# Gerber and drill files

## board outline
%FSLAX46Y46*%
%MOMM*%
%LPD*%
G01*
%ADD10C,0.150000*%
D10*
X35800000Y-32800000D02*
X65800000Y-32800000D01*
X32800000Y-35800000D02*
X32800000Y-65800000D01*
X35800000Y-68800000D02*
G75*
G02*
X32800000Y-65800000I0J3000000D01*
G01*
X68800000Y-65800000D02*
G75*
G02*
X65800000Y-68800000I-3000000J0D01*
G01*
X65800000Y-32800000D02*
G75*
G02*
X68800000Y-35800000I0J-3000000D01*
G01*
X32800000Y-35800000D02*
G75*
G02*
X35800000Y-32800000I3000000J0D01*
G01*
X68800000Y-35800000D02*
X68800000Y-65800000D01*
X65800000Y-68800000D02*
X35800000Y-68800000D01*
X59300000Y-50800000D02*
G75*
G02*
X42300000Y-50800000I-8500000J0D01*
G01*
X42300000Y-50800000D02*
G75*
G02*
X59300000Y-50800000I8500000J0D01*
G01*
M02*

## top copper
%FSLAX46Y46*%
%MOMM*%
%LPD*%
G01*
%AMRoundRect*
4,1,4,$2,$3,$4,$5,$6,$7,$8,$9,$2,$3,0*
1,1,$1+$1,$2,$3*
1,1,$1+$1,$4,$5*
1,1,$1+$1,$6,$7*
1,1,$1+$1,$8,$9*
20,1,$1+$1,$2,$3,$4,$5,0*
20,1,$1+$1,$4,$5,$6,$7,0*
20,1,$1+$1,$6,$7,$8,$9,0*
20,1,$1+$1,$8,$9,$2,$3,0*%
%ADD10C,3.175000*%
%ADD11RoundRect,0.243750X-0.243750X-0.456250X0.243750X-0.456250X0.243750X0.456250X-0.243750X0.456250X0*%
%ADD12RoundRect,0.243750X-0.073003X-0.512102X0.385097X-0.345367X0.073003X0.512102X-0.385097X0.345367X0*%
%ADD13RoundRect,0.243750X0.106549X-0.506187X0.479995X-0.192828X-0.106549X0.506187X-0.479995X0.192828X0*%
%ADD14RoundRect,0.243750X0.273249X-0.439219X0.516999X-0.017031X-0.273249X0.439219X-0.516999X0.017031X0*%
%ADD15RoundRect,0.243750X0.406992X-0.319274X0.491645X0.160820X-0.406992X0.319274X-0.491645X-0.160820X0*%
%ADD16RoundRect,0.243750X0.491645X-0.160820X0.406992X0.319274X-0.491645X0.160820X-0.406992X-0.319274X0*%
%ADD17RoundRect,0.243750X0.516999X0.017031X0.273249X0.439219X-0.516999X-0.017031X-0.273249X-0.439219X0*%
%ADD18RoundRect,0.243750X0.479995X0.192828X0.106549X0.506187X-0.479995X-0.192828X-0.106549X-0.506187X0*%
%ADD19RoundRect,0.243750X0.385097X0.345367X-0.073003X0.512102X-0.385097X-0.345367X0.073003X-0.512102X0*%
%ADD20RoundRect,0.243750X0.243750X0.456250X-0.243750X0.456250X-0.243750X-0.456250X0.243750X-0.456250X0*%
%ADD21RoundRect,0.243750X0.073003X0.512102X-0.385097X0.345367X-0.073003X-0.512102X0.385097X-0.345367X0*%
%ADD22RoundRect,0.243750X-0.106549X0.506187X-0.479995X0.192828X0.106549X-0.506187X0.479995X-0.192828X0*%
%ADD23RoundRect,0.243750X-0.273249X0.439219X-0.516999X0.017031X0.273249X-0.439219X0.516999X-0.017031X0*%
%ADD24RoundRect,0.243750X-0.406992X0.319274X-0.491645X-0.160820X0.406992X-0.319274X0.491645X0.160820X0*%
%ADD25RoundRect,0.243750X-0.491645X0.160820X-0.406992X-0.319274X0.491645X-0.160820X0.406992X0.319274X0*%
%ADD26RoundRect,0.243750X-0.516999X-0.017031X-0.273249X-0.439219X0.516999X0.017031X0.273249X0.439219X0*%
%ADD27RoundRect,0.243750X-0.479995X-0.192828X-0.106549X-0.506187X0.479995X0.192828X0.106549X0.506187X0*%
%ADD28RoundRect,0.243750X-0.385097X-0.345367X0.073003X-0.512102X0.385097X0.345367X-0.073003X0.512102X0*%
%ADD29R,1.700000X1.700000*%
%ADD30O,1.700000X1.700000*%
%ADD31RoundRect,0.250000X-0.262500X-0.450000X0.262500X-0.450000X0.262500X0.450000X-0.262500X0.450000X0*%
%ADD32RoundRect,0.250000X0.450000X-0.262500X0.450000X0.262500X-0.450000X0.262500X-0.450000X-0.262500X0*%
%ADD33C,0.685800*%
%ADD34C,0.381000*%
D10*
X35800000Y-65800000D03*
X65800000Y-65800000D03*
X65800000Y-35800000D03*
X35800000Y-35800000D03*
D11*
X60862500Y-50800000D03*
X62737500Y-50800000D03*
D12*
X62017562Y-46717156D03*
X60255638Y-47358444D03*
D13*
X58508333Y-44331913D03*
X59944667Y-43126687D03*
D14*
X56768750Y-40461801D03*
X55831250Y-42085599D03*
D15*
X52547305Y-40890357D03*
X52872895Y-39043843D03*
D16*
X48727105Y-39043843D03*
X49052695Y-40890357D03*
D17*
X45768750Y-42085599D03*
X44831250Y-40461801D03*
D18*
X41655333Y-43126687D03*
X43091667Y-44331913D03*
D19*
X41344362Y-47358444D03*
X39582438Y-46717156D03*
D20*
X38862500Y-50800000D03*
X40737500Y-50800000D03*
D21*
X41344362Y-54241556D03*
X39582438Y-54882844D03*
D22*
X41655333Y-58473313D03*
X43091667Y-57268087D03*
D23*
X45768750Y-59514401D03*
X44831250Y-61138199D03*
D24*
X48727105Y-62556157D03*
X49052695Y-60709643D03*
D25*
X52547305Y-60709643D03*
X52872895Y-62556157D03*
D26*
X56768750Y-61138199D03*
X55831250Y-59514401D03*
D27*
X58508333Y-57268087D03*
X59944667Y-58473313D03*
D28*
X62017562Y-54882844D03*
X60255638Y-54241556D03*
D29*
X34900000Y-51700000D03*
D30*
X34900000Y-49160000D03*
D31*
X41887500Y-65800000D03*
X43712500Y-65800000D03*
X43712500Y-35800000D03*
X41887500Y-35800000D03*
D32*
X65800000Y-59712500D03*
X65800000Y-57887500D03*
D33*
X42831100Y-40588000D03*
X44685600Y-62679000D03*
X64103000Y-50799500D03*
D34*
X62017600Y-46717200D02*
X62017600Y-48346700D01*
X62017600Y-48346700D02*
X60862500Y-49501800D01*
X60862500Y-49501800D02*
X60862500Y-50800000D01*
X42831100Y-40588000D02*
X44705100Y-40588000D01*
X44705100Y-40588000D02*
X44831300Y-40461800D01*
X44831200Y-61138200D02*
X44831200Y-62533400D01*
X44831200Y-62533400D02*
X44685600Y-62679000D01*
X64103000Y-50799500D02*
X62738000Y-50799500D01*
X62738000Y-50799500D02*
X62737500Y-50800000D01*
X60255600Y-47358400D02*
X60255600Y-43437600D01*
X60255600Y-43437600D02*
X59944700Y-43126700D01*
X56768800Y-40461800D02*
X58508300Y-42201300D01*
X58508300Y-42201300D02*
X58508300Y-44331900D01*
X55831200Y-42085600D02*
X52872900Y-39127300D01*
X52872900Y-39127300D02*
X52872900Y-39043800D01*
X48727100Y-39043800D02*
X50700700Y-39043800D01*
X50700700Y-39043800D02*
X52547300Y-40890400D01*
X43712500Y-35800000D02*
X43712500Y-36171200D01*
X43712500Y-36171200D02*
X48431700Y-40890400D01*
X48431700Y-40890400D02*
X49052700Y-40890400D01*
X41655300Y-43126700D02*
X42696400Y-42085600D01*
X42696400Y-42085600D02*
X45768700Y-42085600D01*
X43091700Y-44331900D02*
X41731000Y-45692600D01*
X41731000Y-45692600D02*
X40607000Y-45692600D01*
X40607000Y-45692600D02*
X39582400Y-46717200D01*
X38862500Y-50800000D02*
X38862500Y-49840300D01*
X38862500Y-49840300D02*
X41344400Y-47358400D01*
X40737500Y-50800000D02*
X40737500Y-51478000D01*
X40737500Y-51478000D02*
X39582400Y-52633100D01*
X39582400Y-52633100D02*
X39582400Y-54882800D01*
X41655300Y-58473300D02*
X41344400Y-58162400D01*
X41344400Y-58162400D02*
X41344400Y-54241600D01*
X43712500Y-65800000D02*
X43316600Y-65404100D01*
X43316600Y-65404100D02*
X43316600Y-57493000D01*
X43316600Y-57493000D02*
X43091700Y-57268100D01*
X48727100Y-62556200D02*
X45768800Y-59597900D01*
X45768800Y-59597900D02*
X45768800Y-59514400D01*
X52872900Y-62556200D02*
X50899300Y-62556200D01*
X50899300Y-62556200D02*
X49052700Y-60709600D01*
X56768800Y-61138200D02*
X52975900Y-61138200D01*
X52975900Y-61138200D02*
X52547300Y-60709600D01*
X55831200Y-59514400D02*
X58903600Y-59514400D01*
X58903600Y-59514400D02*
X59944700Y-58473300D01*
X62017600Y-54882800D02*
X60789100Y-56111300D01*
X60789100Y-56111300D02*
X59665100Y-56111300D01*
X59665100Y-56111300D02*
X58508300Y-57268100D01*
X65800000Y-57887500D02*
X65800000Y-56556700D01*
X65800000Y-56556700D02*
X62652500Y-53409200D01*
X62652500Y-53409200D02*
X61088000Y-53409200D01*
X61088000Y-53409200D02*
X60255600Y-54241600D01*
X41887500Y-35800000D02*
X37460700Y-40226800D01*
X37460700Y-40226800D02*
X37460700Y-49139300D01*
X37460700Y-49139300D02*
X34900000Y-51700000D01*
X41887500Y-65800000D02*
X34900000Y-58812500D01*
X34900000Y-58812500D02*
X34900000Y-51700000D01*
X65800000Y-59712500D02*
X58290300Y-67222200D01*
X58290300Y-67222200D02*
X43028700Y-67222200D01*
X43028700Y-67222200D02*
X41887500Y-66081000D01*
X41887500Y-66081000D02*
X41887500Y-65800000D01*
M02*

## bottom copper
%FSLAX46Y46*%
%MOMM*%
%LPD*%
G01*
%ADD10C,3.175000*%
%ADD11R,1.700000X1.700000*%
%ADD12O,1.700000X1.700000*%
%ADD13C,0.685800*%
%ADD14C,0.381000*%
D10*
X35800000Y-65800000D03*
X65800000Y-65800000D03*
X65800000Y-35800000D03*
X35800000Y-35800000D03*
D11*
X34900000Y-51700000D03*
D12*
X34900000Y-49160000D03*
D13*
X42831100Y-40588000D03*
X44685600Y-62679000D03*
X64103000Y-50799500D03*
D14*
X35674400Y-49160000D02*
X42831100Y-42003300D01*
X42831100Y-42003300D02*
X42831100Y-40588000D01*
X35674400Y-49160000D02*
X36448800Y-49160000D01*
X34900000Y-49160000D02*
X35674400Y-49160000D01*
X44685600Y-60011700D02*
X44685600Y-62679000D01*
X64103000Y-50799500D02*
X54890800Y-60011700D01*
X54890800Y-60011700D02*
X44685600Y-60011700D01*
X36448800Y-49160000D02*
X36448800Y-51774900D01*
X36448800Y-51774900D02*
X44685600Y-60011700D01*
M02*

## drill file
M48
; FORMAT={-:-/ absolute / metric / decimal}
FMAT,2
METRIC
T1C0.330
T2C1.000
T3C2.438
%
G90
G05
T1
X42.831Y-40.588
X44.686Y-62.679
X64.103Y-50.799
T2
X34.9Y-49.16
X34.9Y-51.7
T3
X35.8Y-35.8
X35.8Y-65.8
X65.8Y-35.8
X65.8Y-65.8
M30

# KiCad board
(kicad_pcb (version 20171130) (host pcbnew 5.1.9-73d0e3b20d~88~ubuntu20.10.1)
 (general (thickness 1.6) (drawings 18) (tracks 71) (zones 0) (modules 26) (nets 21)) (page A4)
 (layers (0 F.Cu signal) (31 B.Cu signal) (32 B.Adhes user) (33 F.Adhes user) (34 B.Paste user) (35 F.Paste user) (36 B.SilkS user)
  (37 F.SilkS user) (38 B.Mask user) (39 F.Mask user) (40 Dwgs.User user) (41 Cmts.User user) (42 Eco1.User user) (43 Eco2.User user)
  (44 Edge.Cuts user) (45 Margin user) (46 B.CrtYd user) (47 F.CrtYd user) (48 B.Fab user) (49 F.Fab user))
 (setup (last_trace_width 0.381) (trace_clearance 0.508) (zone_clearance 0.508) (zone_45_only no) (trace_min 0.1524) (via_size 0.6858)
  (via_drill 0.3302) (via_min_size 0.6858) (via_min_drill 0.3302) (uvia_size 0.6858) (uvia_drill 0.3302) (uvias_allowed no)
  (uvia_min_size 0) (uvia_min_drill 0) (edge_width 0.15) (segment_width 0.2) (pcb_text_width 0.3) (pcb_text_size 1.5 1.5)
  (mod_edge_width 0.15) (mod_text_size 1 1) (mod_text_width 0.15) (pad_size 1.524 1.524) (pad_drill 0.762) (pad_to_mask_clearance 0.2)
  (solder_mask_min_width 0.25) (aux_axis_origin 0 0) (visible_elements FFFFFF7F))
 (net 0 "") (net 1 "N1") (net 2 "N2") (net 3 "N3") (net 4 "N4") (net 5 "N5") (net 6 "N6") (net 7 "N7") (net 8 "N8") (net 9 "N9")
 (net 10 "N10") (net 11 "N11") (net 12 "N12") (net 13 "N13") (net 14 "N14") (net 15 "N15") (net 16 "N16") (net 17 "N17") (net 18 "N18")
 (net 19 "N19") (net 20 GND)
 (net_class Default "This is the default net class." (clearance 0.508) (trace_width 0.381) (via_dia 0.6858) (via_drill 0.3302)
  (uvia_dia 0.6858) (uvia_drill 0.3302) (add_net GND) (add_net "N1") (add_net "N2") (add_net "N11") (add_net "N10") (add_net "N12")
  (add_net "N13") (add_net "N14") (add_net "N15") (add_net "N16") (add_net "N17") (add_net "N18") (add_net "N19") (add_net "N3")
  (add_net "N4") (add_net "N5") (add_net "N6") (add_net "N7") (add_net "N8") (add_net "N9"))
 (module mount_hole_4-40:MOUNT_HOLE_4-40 (layer F.Cu) (at 35.8 65.8)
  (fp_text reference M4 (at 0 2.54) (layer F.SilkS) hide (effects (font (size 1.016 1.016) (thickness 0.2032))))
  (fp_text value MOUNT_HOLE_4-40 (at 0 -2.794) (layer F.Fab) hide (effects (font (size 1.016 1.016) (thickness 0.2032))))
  (pad 1 thru_hole circle (at 0 0) (size 3.175 3.175) (drill 2.4384) (layers *.Cu *.Mask)))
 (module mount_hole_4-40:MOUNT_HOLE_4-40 (layer F.Cu) (at 65.8 65.8)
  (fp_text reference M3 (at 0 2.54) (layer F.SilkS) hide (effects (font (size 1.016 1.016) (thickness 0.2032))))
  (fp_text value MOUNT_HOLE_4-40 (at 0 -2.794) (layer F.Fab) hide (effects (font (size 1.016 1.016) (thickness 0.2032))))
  (pad 1 thru_hole circle (at 0 0) (size 3.175 3.175) (drill 2.4384) (layers *.Cu *.Mask)))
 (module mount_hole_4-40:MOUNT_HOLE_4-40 (layer F.Cu) (at 65.8 35.8)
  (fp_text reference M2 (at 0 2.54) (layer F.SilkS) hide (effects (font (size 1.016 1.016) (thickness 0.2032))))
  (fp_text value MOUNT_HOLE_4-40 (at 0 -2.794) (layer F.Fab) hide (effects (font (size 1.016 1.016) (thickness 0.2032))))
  (pad 1 thru_hole circle (at 0 0) (size 3.175 3.175) (drill 2.4384) (layers *.Cu *.Mask)))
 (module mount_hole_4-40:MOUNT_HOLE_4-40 (layer F.Cu) (at 35.8 35.8)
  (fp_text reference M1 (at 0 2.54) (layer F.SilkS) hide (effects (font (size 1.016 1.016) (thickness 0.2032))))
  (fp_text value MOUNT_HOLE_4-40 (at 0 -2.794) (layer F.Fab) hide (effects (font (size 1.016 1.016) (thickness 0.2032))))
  (pad 1 thru_hole circle (at 0 0) (size 3.175 3.175) (drill 2.4384) (layers *.Cu *.Mask)))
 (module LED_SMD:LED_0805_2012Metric (layer F.Cu) (at 61.8 50.8)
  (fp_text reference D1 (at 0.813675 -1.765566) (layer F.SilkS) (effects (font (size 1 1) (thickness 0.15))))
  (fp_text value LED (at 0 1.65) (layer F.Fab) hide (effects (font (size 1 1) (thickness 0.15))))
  (pad 1 smd roundrect (at -0.9375 0) (size 0.975 1.4) (layers F.Cu F.Paste F.Mask) (roundrect_rratio 0.25) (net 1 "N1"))
  (pad 2 smd roundrect (at 0.9375 0) (size 0.975 1.4) (layers F.Cu F.Paste F.Mask) (roundrect_rratio 0.25) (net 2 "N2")))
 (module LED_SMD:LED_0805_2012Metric (layer F.Cu) (at 61.1366 47.0378 20)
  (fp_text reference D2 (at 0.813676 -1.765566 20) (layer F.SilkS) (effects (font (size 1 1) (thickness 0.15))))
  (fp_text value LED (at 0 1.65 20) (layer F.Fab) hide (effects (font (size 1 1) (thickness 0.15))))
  (pad 2 smd roundrect (at 0.9375 0 20) (size 0.975 1.4) (layers F.Cu F.Paste F.Mask) (roundrect_rratio 0.25) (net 1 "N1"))
  (pad 1 smd roundrect (at -0.9375 0 20) (size 0.975 1.4) (layers F.Cu F.Paste F.Mask) (roundrect_rratio 0.25) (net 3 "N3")))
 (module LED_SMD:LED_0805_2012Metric (layer F.Cu) (at 59.2265 43.7293 40)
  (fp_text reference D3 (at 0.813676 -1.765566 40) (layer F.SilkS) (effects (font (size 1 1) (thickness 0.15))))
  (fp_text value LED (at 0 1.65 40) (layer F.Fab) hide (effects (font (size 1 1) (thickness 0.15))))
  (pad 1 smd roundrect (at -0.9375 0 40) (size 0.975 1.4) (layers F.Cu F.Paste F.Mask) (roundrect_rratio 0.25) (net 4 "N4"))
  (pad 2 smd roundrect (at 0.9375 0 40) (size 0.975 1.4) (layers F.Cu F.Paste F.Mask) (roundrect_rratio 0.25) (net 3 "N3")))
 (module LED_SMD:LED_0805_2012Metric (layer F.Cu) (at 56.3 41.2737 60)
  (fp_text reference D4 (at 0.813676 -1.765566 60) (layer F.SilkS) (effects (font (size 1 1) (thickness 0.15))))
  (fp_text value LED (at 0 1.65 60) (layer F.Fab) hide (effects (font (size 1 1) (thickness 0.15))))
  (pad 2 smd roundrect (at 0.9375 0 60) (size 0.975 1.4) (layers F.Cu F.Paste F.Mask) (roundrect_rratio 0.25) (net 4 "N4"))
  (pad 1 smd roundrect (at -0.9375 0 60) (size 0.975 1.4) (layers F.Cu F.Paste F.Mask) (roundrect_rratio 0.25) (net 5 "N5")))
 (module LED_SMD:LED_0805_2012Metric (layer F.Cu) (at 52.7101 39.9671 80)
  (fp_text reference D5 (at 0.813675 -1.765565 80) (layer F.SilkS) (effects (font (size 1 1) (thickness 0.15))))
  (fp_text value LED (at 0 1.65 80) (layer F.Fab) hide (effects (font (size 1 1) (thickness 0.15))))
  (pad 1 smd roundrect (at -0.9375 0 80) (size 0.975 1.4) (layers F.Cu F.Paste F.Mask) (roundrect_rratio 0.25) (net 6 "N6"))
  (pad 2 smd roundrect (at 0.9375 0 80) (size 0.975 1.4) (layers F.Cu F.Paste F.Mask) (roundrect_rratio 0.25) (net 5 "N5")))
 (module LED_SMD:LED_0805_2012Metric (layer F.Cu) (at 48.8899 39.9671 100)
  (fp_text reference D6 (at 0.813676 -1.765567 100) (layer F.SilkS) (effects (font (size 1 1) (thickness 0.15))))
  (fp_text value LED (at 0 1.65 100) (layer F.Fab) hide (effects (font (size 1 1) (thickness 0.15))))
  (pad 2 smd roundrect (at 0.9375 0 100) (size 0.975 1.4) (layers F.Cu F.Paste F.Mask) (roundrect_rratio 0.25) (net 6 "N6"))
  (pad 1 smd roundrect (at -0.9375 0 100) (size 0.975 1.4) (layers F.Cu F.Paste F.Mask) (roundrect_rratio 0.25) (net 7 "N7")))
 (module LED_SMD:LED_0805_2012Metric (layer F.Cu) (at 45.3 41.2737 120)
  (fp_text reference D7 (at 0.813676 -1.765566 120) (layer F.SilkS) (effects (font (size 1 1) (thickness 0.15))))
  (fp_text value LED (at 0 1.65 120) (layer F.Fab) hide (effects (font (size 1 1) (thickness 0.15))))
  (pad 1 smd roundrect (at -0.9375 0 120) (size 0.975 1.4) (layers F.Cu F.Paste F.Mask) (roundrect_rratio 0.25) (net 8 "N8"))
  (pad 2 smd roundrect (at 0.9375 0 120) (size 0.975 1.4) (layers F.Cu F.Paste F.Mask) (roundrect_rratio 0.25) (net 2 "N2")))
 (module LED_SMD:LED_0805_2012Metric (layer F.Cu) (at 42.3735 43.7293 140)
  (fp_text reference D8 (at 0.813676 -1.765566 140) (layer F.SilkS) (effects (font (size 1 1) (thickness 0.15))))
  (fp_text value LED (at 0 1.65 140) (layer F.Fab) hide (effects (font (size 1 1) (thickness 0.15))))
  (pad 2 smd roundrect (at 0.9375 0 140) (size 0.975 1.4) (layers F.Cu F.Paste F.Mask) (roundrect_rratio 0.25) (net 8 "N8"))
  (pad 1 smd roundrect (at -0.9375 0 140) (size 0.975 1.4) (layers F.Cu F.Paste F.Mask) (roundrect_rratio 0.25) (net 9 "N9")))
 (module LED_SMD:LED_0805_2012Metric (layer F.Cu) (at 40.4634 47.0378 160)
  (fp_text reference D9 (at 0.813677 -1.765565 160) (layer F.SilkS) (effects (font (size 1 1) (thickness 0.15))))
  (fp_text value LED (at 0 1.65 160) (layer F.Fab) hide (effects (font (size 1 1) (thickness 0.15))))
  (pad 1 smd roundrect (at -0.9375 0 160) (size 0.975 1.4) (layers F.Cu F.Paste F.Mask) (roundrect_rratio 0.25) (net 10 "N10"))
  (pad 2 smd roundrect (at 0.9375 0 160) (size 0.975 1.4) (layers F.Cu F.Paste F.Mask) (roundrect_rratio 0.25) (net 9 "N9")))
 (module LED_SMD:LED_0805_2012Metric (layer F.Cu) (at 39.8 50.8 180)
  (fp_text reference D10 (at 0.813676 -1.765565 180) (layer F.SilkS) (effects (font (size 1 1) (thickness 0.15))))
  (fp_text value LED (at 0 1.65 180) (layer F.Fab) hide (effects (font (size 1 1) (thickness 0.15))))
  (pad 2 smd roundrect (at 0.9375 0 180) (size 0.975 1.4) (layers F.Cu F.Paste F.Mask) (roundrect_rratio 0.25) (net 10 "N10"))
  (pad 1 smd roundrect (at -0.9375 0 180) (size 0.975 1.4) (layers F.Cu F.Paste F.Mask) (roundrect_rratio 0.25) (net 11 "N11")))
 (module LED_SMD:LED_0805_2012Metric (layer F.Cu) (at 40.4634 54.5622 200)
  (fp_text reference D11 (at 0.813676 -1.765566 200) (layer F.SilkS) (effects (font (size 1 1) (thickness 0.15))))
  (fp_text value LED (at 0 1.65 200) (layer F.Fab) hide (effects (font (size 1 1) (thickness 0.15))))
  (pad 1 smd roundrect (at -0.9375 0 200) (size 0.975 1.4) (layers F.Cu F.Paste F.Mask) (roundrect_rratio 0.25) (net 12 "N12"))
  (pad 2 smd roundrect (at 0.9375 0 200) (size 0.975 1.4) (layers F.Cu F.Paste F.Mask) (roundrect_rratio 0.25) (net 11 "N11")))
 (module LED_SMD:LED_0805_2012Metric (layer F.Cu) (at 42.3735 57.8707 220)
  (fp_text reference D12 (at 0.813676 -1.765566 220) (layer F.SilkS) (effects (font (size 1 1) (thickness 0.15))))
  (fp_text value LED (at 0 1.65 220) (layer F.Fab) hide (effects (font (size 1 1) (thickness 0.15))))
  (pad 2 smd roundrect (at 0.9375 0 220) (size 0.975 1.4) (layers F.Cu F.Paste F.Mask) (roundrect_rratio 0.25) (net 12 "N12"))
  (pad 1 smd roundrect (at -0.9375 0 220) (size 0.975 1.4) (layers F.Cu F.Paste F.Mask) (roundrect_rratio 0.25) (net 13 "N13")))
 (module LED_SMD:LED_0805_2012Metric (layer F.Cu) (at 45.3 60.3263 240)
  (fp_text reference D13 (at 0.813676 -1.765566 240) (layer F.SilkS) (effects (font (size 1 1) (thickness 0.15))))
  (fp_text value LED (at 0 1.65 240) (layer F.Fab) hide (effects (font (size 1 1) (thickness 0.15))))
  (pad 1 smd roundrect (at -0.9375 0 240) (size 0.975 1.4) (layers F.Cu F.Paste F.Mask) (roundrect_rratio 0.25) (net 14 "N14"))
  (pad 2 smd roundrect (at 0.9375 0 240) (size 0.975 1.4) (layers F.Cu F.Paste F.Mask) (roundrect_rratio 0.25) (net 2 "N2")))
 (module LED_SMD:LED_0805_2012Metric (layer F.Cu) (at 48.8899 61.6329 260)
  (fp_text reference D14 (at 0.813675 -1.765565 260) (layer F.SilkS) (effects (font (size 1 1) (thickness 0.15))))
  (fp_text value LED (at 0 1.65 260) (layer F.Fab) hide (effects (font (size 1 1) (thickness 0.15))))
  (pad 2 smd roundrect (at 0.9375 0 260) (size 0.975 1.4) (layers F.Cu F.Paste F.Mask) (roundrect_rratio 0.25) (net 14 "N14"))
  (pad 1 smd roundrect (at -0.9375 0 260) (size 0.975 1.4) (layers F.Cu F.Paste F.Mask) (roundrect_rratio 0.25) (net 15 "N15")))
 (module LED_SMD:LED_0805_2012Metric (layer F.Cu) (at 52.7101 61.6329 280)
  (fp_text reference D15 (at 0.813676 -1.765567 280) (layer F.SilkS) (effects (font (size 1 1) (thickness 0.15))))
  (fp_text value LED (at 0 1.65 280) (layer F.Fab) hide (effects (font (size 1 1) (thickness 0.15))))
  (pad 1 smd roundrect (at -0.9375 0 280) (size 0.975 1.4) (layers F.Cu F.Paste F.Mask) (roundrect_rratio 0.25) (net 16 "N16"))
  (pad 2 smd roundrect (at 0.9375 0 280) (size 0.975 1.4) (layers F.Cu F.Paste F.Mask) (roundrect_rratio 0.25) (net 15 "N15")))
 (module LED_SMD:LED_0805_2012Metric (layer F.Cu) (at 56.3 60.3263 300)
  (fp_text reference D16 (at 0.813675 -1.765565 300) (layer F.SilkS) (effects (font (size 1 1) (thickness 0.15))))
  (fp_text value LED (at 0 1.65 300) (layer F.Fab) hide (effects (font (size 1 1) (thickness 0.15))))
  (pad 2 smd roundrect (at 0.9375 0 300) (size 0.975 1.4) (layers F.Cu F.Paste F.Mask) (roundrect_rratio 0.25) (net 16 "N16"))
  (pad 1 smd roundrect (at -0.9375 0 300) (size 0.975 1.4) (layers F.Cu F.Paste F.Mask) (roundrect_rratio 0.25) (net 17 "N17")))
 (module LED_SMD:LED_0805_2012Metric (layer F.Cu) (at 59.2265 57.8707 320)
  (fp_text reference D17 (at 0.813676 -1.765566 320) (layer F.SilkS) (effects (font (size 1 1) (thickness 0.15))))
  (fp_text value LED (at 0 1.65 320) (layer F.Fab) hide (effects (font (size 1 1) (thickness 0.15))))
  (pad 1 smd roundrect (at -0.9375 0 320) (size 0.975 1.4) (layers F.Cu F.Paste F.Mask) (roundrect_rratio 0.25) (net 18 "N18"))
  (pad 2 smd roundrect (at 0.9375 0 320) (size 0.975 1.4) (layers F.Cu F.Paste F.Mask) (roundrect_rratio 0.25) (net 17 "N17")))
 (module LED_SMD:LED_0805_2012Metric (layer F.Cu) (at 61.1366 54.5622 340)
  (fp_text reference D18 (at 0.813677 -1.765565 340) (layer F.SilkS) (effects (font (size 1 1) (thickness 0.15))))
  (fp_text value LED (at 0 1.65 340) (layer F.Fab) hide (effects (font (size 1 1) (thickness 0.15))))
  (pad 2 smd roundrect (at 0.9375 0 340) (size 0.975 1.4) (layers F.Cu F.Paste F.Mask) (roundrect_rratio 0.25) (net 18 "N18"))
  (pad 1 smd roundrect (at -0.9375 0 340) (size 0.975 1.4) (layers F.Cu F.Paste F.Mask) (roundrect_rratio 0.25) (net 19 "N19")))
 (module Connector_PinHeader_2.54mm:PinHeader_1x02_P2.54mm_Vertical (layer B.Cu) (at 34.9 51.7)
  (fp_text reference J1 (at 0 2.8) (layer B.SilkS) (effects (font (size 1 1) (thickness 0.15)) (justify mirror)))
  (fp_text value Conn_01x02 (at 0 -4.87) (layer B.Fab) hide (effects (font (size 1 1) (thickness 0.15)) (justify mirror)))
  (pad 1 thru_hole rect (at 0 0) (size 1.7 1.7) (drill 1) (layers *.Cu *.Mask) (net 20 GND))
  (pad 2 thru_hole oval (at 0 -2.54) (size 1.7 1.7) (drill 1) (layers *.Cu *.Mask) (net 2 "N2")))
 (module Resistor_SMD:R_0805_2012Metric (layer F.Cu) (at 42.8 65.8)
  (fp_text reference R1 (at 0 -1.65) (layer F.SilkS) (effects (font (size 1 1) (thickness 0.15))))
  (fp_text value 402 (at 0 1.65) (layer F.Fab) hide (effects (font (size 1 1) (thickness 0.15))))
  (pad 1 smd roundrect (at -0.9125 0) (size 1.025 1.4) (layers F.Cu F.Paste F.Mask) (roundrect_rratio 0.243902) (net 20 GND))
  (pad 2 smd roundrect (at 0.9125 0) (size 1.025 1.4) (layers F.Cu F.Paste F.Mask) (roundrect_rratio 0.243902) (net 13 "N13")))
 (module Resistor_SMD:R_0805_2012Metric (layer F.Cu) (at 42.8 35.8)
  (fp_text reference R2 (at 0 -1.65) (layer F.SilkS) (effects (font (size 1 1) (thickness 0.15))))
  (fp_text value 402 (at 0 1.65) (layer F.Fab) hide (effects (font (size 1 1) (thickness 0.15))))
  (pad 2 smd roundrect (at 0.9125 0) (size 1.025 1.4) (layers F.Cu F.Paste F.Mask) (roundrect_rratio 0.243902) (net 7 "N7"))
  (pad 1 smd roundrect (at -0.9125 0) (size 1.025 1.4) (layers F.Cu F.Paste F.Mask) (roundrect_rratio 0.243902) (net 20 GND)))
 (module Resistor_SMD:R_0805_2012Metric (layer F.Cu) (at 65.8 58.8 90)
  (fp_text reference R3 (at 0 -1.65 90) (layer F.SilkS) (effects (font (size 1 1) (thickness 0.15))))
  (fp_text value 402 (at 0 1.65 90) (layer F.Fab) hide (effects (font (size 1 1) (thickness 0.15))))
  (pad 1 smd roundrect (at -0.9125 0 90) (size 1.025 1.4) (layers F.Cu F.Paste F.Mask) (roundrect_rratio 0.243902) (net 20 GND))
  (pad 2 smd roundrect (at 0.9125 0 90) (size 1.025 1.4) (layers F.Cu F.Paste F.Mask) (roundrect_rratio 0.243902) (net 19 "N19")))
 (gr_line (start 35.8 32.8) (end 65.8 32.8) (layer Edge.Cuts) (width 0.15))
 (gr_line (start 32.8 35.8) (end 32.8 65.8) (layer Edge.Cuts) (width 0.15))
 (gr_arc (start 35.8 65.8) (end 32.8 65.8) (angle -90) (layer Edge.Cuts) (width 0.15))
 (gr_arc (start 65.8 65.8) (end 65.8 68.8) (angle -90) (layer Edge.Cuts) (width 0.15))
 (gr_arc (start 65.8 35.8) (end 68.8 35.8) (angle -90) (layer Edge.Cuts) (width 0.15))
 (gr_arc (start 35.8 35.8) (end 35.8 32.8) (angle -90) (layer Edge.Cuts) (width 0.15))
 (gr_line (start 68.8 35.8) (end 68.8 65.8) (layer Edge.Cuts) (width 0.15))
 (gr_line (start 65.8 68.8) (end 35.8 68.8) (layer Edge.Cuts) (width 0.15))
 (gr_circle (center 50.8 50.8) (end 59.3 50.8) (layer Edge.Cuts) (width 0.15))
 (segment (start 62.0176 46.7172) (end 62.0176 48.3467) (width 0.381) (layer F.Cu) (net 1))
 (segment (start 62.0176 48.3467) (end 60.8625 49.5018) (width 0.381) (layer F.Cu) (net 1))
 (segment (start 60.8625 49.5018) (end 60.8625 50.8) (width 0.381) (layer F.Cu) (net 1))
 (segment (start 42.8311 40.588) (end 44.7051 40.588) (width 0.381) (layer F.Cu) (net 2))
 (segment (start 44.7051 40.588) (end 44.8313 40.4618) (width 0.381) (layer F.Cu) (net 2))
 (segment (start 35.6744 49.16) (end 42.8311 42.0033) (width 0.381) (layer B.Cu) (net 2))
 (segment (start 42.8311 42.0033) (end 42.8311 40.588) (width 0.381) (layer B.Cu) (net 2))
 (segment (start 35.6744 49.16) (end 36.4488 49.16) (width 0.381) (layer B.Cu) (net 2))
 (segment (start 34.9 49.16) (end 35.6744 49.16) (width 0.381) (layer B.Cu) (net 2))
 (segment (start 44.6856 60.0117) (end 44.6856 62.679) (width 0.381) (layer B.Cu) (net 2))
 (segment (start 64.103 50.7995) (end 54.8908 60.0117) (width 0.381) (layer B.Cu) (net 2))
 (segment (start 54.8908 60.0117) (end 44.6856 60.0117) (width 0.381) (layer B.Cu) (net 2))
 (segment (start 36.4488 49.16) (end 36.4488 51.7749) (width 0.381) (layer B.Cu) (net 2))
 (segment (start 36.4488 51.7749) (end 44.6856 60.0117) (width 0.381) (layer B.Cu) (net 2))
 (segment (start 44.8312 61.1382) (end 44.8312 62.5334) (width 0.381) (layer F.Cu) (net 2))
 (segment (start 44.8312 62.5334) (end 44.6856 62.679) (width 0.381) (layer F.Cu) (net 2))
 (segment (start 64.103 50.7995) (end 62.738 50.7995) (width 0.381) (layer F.Cu) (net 2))
 (segment (start 62.738 50.7995) (end 62.7375 50.8) (width 0.381) (layer F.Cu) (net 2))
 (via (at 42.8311 40.588) (size 0.6858) (layers F.Cu B.Cu) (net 2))
 (via (at 44.6856 62.679) (size 0.6858) (layers F.Cu B.Cu) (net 2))
 (via (at 64.103 50.7995) (size 0.6858) (layers F.Cu B.Cu) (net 2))
 (segment (start 60.2556 47.3584) (end 60.2556 43.4376) (width 0.381) (layer F.Cu) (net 3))
 (segment (start 60.2556 43.4376) (end 59.9447 43.1267) (width 0.381) (layer F.Cu) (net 3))
 (segment (start 56.7688 40.4618) (end 58.5083 42.2013) (width 0.381) (layer F.Cu) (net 4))
 (segment (start 58.5083 42.2013) (end 58.5083 44.3319) (width 0.381) (layer F.Cu) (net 4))
 (segment (start 55.8312 42.0856) (end 52.8729 39.1273) (width 0.381) (layer F.Cu) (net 5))
 (segment (start 52.8729 39.1273) (end 52.8729 39.0438) (width 0.381) (layer F.Cu) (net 5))
 (segment (start 48.7271 39.0438) (end 50.7007 39.0438) (width 0.381) (layer F.Cu) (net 6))
 (segment (start 50.7007 39.0438) (end 52.5473 40.8904) (width 0.381) (layer F.Cu) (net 6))
 (segment (start 43.7125 35.8) (end 43.7125 36.1712) (width 0.381) (layer F.Cu) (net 7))
 (segment (start 43.7125 36.1712) (end 48.4317 40.8904) (width 0.381) (layer F.Cu) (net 7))
 (segment (start 48.4317 40.8904) (end 49.0527 40.8904) (width 0.381) (layer F.Cu) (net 7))
 (segment (start 41.6553 43.1267) (end 42.6964 42.0856) (width 0.381) (layer F.Cu) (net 8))
 (segment (start 42.6964 42.0856) (end 45.7687 42.0856) (width 0.381) (layer F.Cu) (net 8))
 (segment (start 43.0917 44.3319) (end 41.731 45.6926) (width 0.381) (layer F.Cu) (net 9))
 (segment (start 41.731 45.6926) (end 40.607 45.6926) (width 0.381) (layer F.Cu) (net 9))
 (segment (start 40.607 45.6926) (end 39.5824 46.7172) (width 0.381) (layer F.Cu) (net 9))
 (segment (start 38.8625 50.8) (end 38.8625 49.8403) (width 0.381) (layer F.Cu) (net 10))
 (segment (start 38.8625 49.8403) (end 41.3444 47.3584) (width 0.381) (layer F.Cu) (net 10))
 (segment (start 40.7375 50.8) (end 40.7375 51.478) (width 0.381) (layer F.Cu) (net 11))
 (segment (start 40.7375 51.478) (end 39.5824 52.6331) (width 0.381) (layer F.Cu) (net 11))
 (segment (start 39.5824 52.6331) (end 39.5824 54.8828) (width 0.381) (layer F.Cu) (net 11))
 (segment (start 41.6553 58.4733) (end 41.3444 58.1624) (width 0.381) (layer F.Cu) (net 12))
 (segment (start 41.3444 58.1624) (end 41.3444 54.2416) (width 0.381) (layer F.Cu) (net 12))
 (segment (start 43.7125 65.8) (end 43.3166 65.4041) (width 0.381) (layer F.Cu) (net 13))
 (segment (start 43.3166 65.4041) (end 43.3166 57.493) (width 0.381) (layer F.Cu) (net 13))
 (segment (start 43.3166 57.493) (end 43.0917 57.2681) (width 0.381) (layer F.Cu) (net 13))
 (segment (start 48.7271 62.5562) (end 45.7688 59.5979) (width 0.381) (layer F.Cu) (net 14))
 (segment (start 45.7688 59.5979) (end 45.7688 59.5144) (width 0.381) (layer F.Cu) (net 14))
 (segment (start 52.8729 62.5562) (end 50.8993 62.5562) (width 0.381) (layer F.Cu) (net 15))
 (segment (start 50.8993 62.5562) (end 49.0527 60.7096) (width 0.381) (layer F.Cu) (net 15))
 (segment (start 56.7688 61.1382) (end 52.9759 61.1382) (width 0.381) (layer F.Cu) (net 16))
 (segment (start 52.9759 61.1382) (end 52.5473 60.7096) (width 0.381) (layer F.Cu) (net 16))
 (segment (start 55.8312 59.5144) (end 58.9036 59.5144) (width 0.381) (layer F.Cu) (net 17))
 (segment (start 58.9036 59.5144) (end 59.9447 58.4733) (width 0.381) (layer F.Cu) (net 17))
 (segment (start 62.0176 54.8828) (end 60.7891 56.1113) (width 0.381) (layer F.Cu) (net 18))
 (segment (start 60.7891 56.1113) (end 59.6651 56.1113) (width 0.381) (layer F.Cu) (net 18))
 (segment (start 59.6651 56.1113) (end 58.5083 57.2681) (width 0.381) (layer F.Cu) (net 18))
 (segment (start 65.8 57.8875) (end 65.8 56.5567) (width 0.381) (layer F.Cu) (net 19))
 (segment (start 65.8 56.5567) (end 62.6525 53.4092) (width 0.381) (layer F.Cu) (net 19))
 (segment (start 62.6525 53.4092) (end 61.088 53.4092) (width 0.381) (layer F.Cu) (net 19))
 (segment (start 61.088 53.4092) (end 60.2556 54.2416) (width 0.381) (layer F.Cu) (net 19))
 (segment (start 41.8875 35.8) (end 37.4607 40.2268) (width 0.381) (layer F.Cu) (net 20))
 (segment (start 37.4607 40.2268) (end 37.4607 49.1393) (width 0.381) (layer F.Cu) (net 20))
 (segment (start 37.4607 49.1393) (end 34.9 51.7) (width 0.381) (layer F.Cu) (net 20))
 (segment (start 41.8875 65.8) (end 34.9 58.8125) (width 0.381) (layer F.Cu) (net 20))
 (segment (start 34.9 58.8125) (end 34.9 51.7) (width 0.381) (layer F.Cu) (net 20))
 (segment (start 65.8 59.7125) (end 58.2903 67.2222) (width 0.381) (layer F.Cu) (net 20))
 (segment (start 58.2903 67.2222) (end 43.0287 67.2222) (width 0.381) (layer F.Cu) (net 20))
 (segment (start 43.0287 67.2222) (end 41.8875 66.081) (width 0.381) (layer F.Cu) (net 20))
 (segment (start 41.8875 66.081) (end 41.8875 65.8) (width 0.381) (layer F.Cu) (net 20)))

